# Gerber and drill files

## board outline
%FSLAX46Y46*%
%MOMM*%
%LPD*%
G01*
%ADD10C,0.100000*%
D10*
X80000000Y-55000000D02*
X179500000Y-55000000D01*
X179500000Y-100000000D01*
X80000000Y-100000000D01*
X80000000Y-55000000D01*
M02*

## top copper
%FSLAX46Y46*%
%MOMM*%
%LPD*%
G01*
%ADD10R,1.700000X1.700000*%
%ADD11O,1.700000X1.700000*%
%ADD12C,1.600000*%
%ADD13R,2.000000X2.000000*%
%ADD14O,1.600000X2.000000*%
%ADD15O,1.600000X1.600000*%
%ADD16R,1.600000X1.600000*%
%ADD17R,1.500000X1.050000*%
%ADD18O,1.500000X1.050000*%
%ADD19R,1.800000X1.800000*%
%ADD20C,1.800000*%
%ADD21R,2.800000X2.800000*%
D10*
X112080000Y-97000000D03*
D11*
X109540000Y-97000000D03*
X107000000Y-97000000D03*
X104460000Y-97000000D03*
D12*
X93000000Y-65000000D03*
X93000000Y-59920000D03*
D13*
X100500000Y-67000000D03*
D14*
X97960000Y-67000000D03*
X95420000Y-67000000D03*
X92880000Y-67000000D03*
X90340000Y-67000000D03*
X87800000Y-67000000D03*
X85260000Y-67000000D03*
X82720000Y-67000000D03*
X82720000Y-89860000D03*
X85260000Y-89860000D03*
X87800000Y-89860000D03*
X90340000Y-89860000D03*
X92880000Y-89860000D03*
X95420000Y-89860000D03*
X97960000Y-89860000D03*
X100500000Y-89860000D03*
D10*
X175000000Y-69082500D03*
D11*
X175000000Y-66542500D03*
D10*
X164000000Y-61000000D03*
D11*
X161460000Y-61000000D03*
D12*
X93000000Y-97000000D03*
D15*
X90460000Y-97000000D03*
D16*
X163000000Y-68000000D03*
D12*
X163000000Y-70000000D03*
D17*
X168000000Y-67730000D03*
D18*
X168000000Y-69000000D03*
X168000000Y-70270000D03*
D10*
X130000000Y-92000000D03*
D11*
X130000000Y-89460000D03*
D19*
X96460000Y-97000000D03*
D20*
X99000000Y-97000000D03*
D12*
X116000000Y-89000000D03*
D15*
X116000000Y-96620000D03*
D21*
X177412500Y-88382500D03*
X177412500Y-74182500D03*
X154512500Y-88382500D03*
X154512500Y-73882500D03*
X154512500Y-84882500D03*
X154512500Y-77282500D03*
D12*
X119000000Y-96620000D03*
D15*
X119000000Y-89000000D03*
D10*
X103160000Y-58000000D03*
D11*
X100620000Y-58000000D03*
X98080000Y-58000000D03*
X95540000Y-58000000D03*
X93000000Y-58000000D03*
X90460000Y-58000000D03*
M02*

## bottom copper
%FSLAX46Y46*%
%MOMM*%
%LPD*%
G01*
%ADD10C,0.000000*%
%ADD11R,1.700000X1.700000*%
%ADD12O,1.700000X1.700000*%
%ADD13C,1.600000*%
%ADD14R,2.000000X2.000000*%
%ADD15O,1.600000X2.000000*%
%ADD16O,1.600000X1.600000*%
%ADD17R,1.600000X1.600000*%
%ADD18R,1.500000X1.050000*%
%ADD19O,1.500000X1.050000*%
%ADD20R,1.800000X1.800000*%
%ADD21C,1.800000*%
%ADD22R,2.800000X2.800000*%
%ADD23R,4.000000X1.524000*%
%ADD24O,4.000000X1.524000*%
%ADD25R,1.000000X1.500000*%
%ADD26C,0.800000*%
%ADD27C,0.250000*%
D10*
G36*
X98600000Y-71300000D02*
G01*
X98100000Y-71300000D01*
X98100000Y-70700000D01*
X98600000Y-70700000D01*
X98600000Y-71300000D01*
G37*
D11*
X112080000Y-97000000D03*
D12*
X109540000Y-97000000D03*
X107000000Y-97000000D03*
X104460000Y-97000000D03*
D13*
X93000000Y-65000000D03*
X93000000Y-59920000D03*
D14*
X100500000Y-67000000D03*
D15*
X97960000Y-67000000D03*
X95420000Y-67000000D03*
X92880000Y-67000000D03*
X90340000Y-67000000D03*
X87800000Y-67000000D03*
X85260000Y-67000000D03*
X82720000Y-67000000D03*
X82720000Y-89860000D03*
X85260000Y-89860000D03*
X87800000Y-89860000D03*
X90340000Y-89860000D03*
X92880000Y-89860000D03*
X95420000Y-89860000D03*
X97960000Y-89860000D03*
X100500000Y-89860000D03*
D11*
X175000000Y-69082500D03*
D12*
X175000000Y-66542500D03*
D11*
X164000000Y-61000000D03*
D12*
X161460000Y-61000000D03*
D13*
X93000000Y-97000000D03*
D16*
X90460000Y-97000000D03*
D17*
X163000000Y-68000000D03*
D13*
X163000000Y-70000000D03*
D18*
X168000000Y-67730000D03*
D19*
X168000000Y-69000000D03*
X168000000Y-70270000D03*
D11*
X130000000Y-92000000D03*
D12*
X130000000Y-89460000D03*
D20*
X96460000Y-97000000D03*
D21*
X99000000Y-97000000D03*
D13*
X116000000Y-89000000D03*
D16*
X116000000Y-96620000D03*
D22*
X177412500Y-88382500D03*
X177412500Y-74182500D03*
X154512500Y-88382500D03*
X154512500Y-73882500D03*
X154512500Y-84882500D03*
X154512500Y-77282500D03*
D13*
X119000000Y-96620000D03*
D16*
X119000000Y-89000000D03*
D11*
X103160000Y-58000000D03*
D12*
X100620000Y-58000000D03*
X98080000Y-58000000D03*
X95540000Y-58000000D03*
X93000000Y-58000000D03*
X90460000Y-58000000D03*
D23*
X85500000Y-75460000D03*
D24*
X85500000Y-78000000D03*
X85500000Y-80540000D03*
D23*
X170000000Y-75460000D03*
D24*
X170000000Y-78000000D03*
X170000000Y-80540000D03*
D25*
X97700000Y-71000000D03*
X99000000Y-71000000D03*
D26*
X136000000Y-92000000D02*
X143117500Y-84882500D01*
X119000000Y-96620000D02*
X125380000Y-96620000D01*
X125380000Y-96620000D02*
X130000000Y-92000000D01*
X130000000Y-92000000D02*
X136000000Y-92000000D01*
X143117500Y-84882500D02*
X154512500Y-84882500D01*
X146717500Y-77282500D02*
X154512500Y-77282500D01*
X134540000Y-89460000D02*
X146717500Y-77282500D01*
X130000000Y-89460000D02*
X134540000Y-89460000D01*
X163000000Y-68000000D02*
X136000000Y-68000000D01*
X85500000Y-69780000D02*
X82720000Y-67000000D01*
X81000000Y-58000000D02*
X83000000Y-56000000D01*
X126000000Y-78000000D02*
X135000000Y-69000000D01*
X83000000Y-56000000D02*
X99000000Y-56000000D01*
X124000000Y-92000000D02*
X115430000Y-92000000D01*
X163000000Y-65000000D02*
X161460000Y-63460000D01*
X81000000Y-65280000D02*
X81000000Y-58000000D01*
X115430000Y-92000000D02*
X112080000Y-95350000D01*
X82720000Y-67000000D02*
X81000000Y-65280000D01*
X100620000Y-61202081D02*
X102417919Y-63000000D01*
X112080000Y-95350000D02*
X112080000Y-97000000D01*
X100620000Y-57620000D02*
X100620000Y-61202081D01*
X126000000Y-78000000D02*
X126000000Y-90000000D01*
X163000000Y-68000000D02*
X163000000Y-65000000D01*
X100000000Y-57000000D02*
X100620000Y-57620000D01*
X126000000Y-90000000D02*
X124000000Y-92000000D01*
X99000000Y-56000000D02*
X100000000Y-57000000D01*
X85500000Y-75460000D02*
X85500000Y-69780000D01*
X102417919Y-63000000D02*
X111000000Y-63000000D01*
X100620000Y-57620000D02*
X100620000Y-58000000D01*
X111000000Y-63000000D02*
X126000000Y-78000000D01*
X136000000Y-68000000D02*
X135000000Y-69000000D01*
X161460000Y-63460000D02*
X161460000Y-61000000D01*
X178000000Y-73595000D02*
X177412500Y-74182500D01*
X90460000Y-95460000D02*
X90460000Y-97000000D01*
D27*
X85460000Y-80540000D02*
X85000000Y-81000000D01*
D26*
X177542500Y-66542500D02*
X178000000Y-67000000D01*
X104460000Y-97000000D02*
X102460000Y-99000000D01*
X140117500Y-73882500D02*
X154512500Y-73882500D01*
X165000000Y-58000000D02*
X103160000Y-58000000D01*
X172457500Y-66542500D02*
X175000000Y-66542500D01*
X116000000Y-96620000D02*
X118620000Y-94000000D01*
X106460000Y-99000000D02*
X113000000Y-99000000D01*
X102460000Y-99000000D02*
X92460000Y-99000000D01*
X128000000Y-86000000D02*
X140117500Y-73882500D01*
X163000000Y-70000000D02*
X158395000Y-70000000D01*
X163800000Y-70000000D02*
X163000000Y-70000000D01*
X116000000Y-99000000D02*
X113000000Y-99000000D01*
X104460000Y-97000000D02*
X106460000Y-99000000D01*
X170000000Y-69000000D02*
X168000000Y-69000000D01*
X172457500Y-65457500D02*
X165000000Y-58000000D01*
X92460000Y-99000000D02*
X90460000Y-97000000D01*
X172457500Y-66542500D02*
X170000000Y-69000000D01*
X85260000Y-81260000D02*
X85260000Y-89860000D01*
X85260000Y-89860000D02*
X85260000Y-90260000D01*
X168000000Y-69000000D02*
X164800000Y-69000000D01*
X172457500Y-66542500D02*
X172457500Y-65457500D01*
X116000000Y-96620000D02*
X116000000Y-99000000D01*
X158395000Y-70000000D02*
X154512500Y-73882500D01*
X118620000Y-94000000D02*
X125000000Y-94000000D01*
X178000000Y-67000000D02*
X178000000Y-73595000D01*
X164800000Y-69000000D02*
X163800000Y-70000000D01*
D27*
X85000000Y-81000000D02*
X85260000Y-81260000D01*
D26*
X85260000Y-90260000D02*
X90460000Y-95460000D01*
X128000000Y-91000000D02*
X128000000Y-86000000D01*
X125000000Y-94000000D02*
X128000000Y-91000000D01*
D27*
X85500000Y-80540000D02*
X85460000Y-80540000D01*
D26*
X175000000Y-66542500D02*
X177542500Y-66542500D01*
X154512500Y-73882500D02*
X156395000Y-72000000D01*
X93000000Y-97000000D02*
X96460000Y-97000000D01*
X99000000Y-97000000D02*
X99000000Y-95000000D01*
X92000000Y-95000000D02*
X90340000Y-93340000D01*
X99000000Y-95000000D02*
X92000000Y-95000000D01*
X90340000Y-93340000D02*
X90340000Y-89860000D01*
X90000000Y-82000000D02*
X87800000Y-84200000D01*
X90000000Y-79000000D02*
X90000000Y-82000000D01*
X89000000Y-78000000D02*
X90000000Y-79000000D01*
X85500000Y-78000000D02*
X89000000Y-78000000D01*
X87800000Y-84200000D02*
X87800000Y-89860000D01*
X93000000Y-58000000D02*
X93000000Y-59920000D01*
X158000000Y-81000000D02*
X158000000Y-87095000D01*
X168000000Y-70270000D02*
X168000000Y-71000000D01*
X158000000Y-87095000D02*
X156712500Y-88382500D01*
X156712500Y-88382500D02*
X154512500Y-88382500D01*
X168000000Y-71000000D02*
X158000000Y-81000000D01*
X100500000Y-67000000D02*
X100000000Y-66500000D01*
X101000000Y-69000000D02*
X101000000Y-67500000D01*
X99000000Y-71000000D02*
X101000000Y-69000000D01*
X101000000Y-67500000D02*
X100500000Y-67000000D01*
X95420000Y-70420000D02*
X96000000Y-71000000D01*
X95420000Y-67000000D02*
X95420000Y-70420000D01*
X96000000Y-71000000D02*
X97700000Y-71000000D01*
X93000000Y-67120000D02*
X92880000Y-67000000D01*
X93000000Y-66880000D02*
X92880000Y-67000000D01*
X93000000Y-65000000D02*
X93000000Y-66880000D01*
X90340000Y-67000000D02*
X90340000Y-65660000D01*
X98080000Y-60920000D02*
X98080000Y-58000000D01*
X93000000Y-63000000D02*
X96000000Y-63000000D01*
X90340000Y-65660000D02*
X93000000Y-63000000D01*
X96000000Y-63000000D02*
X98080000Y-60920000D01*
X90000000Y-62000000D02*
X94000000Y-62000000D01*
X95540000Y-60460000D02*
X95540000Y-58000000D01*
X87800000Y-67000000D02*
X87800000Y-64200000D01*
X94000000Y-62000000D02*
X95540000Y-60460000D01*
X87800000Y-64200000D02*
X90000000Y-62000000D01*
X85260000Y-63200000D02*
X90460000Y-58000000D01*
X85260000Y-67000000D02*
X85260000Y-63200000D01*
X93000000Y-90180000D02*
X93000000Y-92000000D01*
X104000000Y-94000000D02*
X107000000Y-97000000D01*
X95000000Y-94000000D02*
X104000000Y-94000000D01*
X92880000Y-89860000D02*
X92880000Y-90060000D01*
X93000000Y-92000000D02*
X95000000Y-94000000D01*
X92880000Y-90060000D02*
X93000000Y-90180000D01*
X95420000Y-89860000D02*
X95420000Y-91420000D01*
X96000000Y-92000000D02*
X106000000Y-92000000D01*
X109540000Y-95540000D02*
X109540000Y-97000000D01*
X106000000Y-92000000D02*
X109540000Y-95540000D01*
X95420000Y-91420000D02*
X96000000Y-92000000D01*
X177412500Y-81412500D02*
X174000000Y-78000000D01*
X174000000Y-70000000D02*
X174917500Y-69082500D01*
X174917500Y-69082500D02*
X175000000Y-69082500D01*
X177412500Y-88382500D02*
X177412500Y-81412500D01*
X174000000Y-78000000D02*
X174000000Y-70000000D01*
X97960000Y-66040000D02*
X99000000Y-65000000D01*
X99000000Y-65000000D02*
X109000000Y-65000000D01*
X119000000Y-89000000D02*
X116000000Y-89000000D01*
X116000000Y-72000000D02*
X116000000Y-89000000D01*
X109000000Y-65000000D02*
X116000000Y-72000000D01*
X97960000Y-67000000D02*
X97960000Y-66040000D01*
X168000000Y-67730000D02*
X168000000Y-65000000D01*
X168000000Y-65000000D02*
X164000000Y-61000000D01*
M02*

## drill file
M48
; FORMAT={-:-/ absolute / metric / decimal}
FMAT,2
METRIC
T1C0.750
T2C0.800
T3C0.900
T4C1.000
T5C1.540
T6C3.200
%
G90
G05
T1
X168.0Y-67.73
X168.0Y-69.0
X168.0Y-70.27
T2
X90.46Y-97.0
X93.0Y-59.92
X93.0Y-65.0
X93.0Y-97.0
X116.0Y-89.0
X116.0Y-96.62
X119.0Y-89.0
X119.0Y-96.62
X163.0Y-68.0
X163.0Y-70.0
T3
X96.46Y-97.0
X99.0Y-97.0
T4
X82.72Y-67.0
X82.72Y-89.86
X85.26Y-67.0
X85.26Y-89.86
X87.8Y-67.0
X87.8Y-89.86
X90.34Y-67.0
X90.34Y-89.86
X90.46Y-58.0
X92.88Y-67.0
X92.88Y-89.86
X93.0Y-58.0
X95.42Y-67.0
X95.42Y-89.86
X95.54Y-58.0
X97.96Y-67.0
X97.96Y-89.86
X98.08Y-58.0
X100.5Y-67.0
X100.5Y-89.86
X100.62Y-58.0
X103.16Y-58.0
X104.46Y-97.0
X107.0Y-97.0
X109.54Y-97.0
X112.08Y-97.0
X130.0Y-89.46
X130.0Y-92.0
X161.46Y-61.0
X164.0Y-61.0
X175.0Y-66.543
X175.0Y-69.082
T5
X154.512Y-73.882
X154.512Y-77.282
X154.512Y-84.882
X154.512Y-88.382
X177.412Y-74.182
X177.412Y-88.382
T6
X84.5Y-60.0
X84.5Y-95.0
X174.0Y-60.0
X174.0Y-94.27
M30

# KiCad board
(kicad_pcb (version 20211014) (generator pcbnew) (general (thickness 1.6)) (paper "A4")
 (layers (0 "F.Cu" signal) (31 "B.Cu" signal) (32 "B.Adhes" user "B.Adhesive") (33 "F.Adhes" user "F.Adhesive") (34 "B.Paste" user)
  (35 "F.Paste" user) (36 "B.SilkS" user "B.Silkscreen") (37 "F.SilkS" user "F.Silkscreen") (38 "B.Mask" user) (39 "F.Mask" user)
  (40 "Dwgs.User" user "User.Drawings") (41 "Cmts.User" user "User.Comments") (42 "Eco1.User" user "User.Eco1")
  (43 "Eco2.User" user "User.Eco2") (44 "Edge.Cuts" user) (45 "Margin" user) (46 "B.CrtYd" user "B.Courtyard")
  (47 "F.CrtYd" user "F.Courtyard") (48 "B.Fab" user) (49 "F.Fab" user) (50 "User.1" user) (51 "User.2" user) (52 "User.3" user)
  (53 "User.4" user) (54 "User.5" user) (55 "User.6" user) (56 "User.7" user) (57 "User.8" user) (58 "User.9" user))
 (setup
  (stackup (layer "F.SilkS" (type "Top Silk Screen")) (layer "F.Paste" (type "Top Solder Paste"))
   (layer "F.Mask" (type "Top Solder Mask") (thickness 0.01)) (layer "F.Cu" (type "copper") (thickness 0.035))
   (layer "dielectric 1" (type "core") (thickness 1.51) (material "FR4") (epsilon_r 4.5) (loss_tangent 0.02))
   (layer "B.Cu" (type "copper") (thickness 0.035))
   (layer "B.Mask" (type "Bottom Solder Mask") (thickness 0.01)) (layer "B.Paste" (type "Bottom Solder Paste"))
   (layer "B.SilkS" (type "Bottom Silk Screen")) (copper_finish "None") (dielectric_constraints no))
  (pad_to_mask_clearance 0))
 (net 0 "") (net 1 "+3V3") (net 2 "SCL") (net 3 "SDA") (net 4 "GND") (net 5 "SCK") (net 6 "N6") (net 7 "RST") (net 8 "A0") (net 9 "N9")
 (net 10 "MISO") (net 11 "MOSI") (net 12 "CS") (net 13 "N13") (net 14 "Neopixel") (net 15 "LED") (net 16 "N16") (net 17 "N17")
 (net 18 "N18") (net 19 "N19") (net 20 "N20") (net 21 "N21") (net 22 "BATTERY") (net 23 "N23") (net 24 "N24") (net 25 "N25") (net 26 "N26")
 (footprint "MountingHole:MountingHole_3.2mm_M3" (layer "F.Cu") (at 174 60)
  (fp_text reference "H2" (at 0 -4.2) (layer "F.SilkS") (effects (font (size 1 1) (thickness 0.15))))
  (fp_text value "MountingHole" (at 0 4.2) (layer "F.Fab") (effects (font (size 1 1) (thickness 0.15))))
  (pad "" np_thru_hole circle (at 0 0) (size 3.2 3.2) (drill 3.2) (layers *.Cu *.Mask)))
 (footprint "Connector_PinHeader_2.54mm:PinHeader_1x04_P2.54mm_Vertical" (layer "F.Cu") (at 112.08 97 -90)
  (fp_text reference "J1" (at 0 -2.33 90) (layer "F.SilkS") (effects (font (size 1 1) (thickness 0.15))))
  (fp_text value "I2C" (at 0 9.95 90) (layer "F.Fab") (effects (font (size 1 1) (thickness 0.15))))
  (pad "1" thru_hole rect (at 0 0 270) (size 1.7 1.7) (drill 1) (layers *.Cu *.Mask) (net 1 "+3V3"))
  (pad "2" thru_hole oval (at 0 2.54 270) (size 1.7 1.7) (drill 1) (layers *.Cu *.Mask) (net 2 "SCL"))
  (pad "3" thru_hole oval (at 0 5.08 270) (size 1.7 1.7) (drill 1) (layers *.Cu *.Mask) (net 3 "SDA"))
  (pad "4" thru_hole oval (at 0 7.62 270) (size 1.7 1.7) (drill 1) (layers *.Cu *.Mask) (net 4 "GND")))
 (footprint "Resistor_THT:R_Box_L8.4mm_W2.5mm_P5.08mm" (layer "F.Cu") (at 93 65 90)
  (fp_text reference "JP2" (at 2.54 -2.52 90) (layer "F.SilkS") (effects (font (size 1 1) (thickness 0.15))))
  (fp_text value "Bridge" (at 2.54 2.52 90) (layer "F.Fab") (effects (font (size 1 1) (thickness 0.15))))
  (pad "1" thru_hole circle (at 0 0 90) (size 1.6 1.6) (drill 0.8) (layers *.Cu *.Mask) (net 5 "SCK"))
  (pad "2" thru_hole circle (at 5.08 0 90) (size 1.6 1.6) (drill 0.8) (layers *.Cu *.Mask) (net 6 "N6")))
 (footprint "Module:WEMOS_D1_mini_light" (layer "F.Cu") (at 100.5 67 -90)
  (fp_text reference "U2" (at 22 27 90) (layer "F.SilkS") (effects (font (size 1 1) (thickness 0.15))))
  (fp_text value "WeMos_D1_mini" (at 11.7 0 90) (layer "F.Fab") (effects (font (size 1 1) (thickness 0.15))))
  (pad "1" thru_hole rect (at 0 0 270) (size 2 2) (drill 1) (layers *.Cu *.Mask) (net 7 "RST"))
  (pad "2" thru_hole oval (at 0 2.54 270) (size 2 1.6) (drill 1) (layers *.Cu *.Mask) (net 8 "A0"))
  (pad "3" thru_hole oval (at 0 5.08 270) (size 2 1.6) (drill 1) (layers *.Cu *.Mask) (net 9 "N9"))
  (pad "4" thru_hole oval (at 0 7.62 270) (size 2 1.6) (drill 1) (layers *.Cu *.Mask) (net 5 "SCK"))
  (pad "5" thru_hole oval (at 0 10.16 270) (size 2 1.6) (drill 1) (layers *.Cu *.Mask) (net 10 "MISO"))
  (pad "6" thru_hole oval (at 0 12.7 270) (size 2 1.6) (drill 1) (layers *.Cu *.Mask) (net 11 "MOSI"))
  (pad "7" thru_hole oval (at 0 15.24 270) (size 2 1.6) (drill 1) (layers *.Cu *.Mask) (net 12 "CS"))
  (pad "8" thru_hole oval (at 0 17.78 270) (size 2 1.6) (drill 1) (layers *.Cu *.Mask) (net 1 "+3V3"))
  (pad "9" thru_hole oval (at 22.86 17.78 270) (size 2 1.6) (drill 1) (layers *.Cu *.Mask) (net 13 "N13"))
  (pad "10" thru_hole oval (at 22.86 15.24 270) (size 2 1.6) (drill 1) (layers *.Cu *.Mask) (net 4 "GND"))
  (pad "11" thru_hole oval (at 22.86 12.7 270) (size 2 1.6) (drill 1) (layers *.Cu *.Mask) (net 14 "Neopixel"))
  (pad "12" thru_hole oval (at 22.86 10.16 270) (size 2 1.6) (drill 1) (layers *.Cu *.Mask) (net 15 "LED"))
  (pad "13" thru_hole oval (at 22.86 7.62 270) (size 2 1.6) (drill 1) (layers *.Cu *.Mask) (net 3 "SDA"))
  (pad "14" thru_hole oval (at 22.86 5.08 270) (size 2 1.6) (drill 1) (layers *.Cu *.Mask) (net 2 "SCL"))
  (pad "15" thru_hole oval (at 22.86 2.54 270) (size 2 1.6) (drill 1) (layers *.Cu *.Mask) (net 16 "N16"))
  (pad "16" thru_hole oval (at 22.86 0 270) (size 2 1.6) (drill 1) (layers *.Cu *.Mask) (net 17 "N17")))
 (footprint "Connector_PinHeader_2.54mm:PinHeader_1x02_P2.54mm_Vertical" (layer "F.Cu") (at 175 69.0825 180)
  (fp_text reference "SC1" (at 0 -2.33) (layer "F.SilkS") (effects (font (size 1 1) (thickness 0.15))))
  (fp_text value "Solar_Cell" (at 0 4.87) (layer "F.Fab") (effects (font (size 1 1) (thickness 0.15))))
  (pad "1" thru_hole rect (at 0 0 180) (size 1.7 1.7) (drill 1) (layers *.Cu *.Mask) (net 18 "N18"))
  (pad "2" thru_hole oval (at 0 2.54 180) (size 1.7 1.7) (drill 1) (layers *.Cu *.Mask) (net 4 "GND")))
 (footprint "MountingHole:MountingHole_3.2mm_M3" (layer "F.Cu") (at 84.5 95)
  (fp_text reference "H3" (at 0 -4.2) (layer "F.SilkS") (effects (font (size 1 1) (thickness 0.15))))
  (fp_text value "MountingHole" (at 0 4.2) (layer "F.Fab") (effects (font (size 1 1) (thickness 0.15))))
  (pad "" np_thru_hole circle (at 0 0) (size 3.2 3.2) (drill 3.2) (layers *.Cu *.Mask)))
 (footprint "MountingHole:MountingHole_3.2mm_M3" (layer "F.Cu") (at 174 94.27)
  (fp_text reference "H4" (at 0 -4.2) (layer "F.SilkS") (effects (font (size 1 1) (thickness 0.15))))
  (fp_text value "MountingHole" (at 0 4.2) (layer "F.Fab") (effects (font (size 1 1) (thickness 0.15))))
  (pad "" np_thru_hole circle (at 0 0) (size 3.2 3.2) (drill 3.2) (layers *.Cu *.Mask)))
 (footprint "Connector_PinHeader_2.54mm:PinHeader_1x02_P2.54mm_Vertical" (layer "F.Cu") (at 164 61 -90)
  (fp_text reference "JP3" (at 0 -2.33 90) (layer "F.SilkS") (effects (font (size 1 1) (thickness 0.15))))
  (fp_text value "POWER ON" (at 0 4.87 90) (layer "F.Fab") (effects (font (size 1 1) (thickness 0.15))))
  (pad "1" thru_hole rect (at 0 0 270) (size 1.7 1.7) (drill 1) (layers *.Cu *.Mask) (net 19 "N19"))
  (pad "2" thru_hole oval (at 0 2.54 270) (size 1.7 1.7) (drill 1) (layers *.Cu *.Mask) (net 1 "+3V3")))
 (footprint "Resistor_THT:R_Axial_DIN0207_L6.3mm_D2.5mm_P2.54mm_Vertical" (layer "F.Cu") (at 93 97 180)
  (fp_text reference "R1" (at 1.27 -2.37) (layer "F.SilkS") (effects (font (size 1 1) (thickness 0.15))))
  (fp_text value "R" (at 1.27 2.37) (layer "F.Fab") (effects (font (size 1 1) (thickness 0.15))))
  (pad "1" thru_hole circle (at 0 0 180) (size 1.6 1.6) (drill 0.8) (layers *.Cu *.Mask) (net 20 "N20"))
  (pad "2" thru_hole oval (at 2.54 0 180) (size 1.6 1.6) (drill 0.8) (layers *.Cu *.Mask) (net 4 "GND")))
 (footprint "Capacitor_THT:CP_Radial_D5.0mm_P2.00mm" (layer "F.Cu") (at 163 68 -90)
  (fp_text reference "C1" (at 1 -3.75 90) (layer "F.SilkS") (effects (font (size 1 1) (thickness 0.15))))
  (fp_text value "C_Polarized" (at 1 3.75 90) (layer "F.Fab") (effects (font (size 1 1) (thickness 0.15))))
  (pad "1" thru_hole rect (at 0 0 270) (size 1.6 1.6) (drill 0.8) (layers *.Cu *.Mask) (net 1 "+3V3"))
  (pad "2" thru_hole circle (at 2 0 270) (size 1.6 1.6) (drill 0.8) (layers *.Cu *.Mask) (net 4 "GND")))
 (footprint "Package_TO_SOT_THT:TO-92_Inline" (layer "F.Cu") (at 168 67.73 -90)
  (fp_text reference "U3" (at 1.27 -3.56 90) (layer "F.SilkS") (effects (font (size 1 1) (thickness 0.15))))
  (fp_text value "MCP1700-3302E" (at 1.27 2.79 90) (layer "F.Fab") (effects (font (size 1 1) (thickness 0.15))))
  (pad "1" thru_hole rect (at 0 0 270) (size 1.05 1.5) (drill 0.75) (layers *.Cu *.Mask) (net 19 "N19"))
  (pad "2" thru_hole oval (at 1.27 0 270) (size 1.05 1.5) (drill 0.75) (layers *.Cu *.Mask) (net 4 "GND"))
  (pad "3" thru_hole oval (at 2.54 0 270) (size 1.05 1.5) (drill 0.75) (layers *.Cu *.Mask) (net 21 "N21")))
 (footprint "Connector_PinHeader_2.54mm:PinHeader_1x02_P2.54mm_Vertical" (layer "F.Cu") (at 130 92 180)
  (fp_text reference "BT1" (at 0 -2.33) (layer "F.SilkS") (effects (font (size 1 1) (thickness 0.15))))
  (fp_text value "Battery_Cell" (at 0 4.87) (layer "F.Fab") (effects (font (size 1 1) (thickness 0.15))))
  (pad "1" thru_hole rect (at 0 0 180) (size 1.7 1.7) (drill 1) (layers *.Cu *.Mask) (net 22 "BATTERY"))
  (pad "2" thru_hole oval (at 0 2.54 180) (size 1.7 1.7) (drill 1) (layers *.Cu *.Mask) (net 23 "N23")))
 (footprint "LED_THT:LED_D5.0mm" (layer "F.Cu") (at 96.46 97)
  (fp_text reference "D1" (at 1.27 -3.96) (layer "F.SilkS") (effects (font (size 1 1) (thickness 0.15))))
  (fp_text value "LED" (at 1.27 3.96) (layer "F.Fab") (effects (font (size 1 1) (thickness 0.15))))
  (pad "1" thru_hole rect (at 0 0) (size 1.8 1.8) (drill 0.9) (layers *.Cu *.Mask) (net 20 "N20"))
  (pad "2" thru_hole circle (at 2.54 0) (size 1.8 1.8) (drill 0.9) (layers *.Cu *.Mask) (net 15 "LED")))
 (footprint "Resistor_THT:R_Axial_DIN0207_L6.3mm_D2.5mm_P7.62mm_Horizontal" (layer "F.Cu") (at 116 89 -90)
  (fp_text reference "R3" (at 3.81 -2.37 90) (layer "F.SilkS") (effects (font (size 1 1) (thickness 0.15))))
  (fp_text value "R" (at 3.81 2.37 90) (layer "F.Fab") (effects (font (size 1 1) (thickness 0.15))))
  (pad "1" thru_hole circle (at 0 0 270) (size 1.6 1.6) (drill 0.8) (layers *.Cu *.Mask) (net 8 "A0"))
  (pad "2" thru_hole oval (at 7.62 0 270) (size 1.6 1.6) (drill 0.8) (layers *.Cu *.Mask) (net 4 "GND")))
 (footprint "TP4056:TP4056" (layer "F.Cu") (at 179.1125 90.0825 180)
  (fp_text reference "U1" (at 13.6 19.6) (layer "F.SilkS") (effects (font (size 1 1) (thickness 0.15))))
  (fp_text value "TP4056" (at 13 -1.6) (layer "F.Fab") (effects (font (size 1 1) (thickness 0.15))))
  (pad "1" thru_hole rect locked (at 1.7 1.7 180) (size 2.8 2.8) (drill 1.54) (layers *.Cu *.Mask) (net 18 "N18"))
  (pad "2" thru_hole rect locked (at 1.7 15.9 180) (size 2.8 2.8) (drill 1.54) (layers *.Cu *.Mask) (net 4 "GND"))
  (pad "3" thru_hole rect locked (at 24.6 1.7 180) (size 2.8 2.8) (drill 1.54) (layers *.Cu *.Mask) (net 21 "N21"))
  (pad "4" thru_hole rect locked (at 24.6 16.2 180) (size 2.8 2.8) (drill 1.54) (layers *.Cu *.Mask) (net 4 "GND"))
  (pad "5" thru_hole rect locked (at 24.6 5.2 180) (size 2.8 2.8) (drill 1.54) (layers *.Cu *.Mask) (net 22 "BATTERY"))
  (pad "6" thru_hole rect locked (at 24.6 12.8 180) (size 2.8 2.8) (drill 1.54) (layers *.Cu *.Mask) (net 23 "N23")))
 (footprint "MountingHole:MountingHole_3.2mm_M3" (layer "F.Cu") (at 84.5 60)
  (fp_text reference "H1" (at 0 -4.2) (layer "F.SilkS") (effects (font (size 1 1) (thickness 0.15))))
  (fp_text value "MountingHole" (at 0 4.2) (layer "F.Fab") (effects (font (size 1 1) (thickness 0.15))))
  (pad "" np_thru_hole circle (at 0 0) (size 3.2 3.2) (drill 3.2) (layers *.Cu *.Mask)))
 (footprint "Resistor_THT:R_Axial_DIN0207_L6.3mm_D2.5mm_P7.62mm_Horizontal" (layer "F.Cu") (at 119 96.62 90)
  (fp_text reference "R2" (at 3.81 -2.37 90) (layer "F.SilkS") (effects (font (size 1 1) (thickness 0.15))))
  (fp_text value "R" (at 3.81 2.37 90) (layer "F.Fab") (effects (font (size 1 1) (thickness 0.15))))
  (pad "1" thru_hole circle (at 0 0 90) (size 1.6 1.6) (drill 0.8) (layers *.Cu *.Mask) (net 22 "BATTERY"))
  (pad "2" thru_hole oval (at 7.62 0 90) (size 1.6 1.6) (drill 0.8) (layers *.Cu *.Mask) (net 8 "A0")))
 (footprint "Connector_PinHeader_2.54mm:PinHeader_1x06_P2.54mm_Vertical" (layer "F.Cu") (at 103.16 58 -90)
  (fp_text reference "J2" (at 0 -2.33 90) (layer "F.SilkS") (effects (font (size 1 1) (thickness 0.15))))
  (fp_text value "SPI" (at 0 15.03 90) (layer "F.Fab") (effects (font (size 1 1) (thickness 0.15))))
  (pad "1" thru_hole rect (at 0 0 270) (size 1.7 1.7) (drill 1) (layers *.Cu *.Mask) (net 4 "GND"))
  (pad "2" thru_hole oval (at 0 2.54 270) (size 1.7 1.7) (drill 1) (layers *.Cu *.Mask) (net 1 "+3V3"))
  (pad "3" thru_hole oval (at 0 5.08 270) (size 1.7 1.7) (drill 1) (layers *.Cu *.Mask) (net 10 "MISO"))
  (pad "4" thru_hole oval (at 0 7.62 270) (size 1.7 1.7) (drill 1) (layers *.Cu *.Mask) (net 11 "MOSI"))
  (pad "5" thru_hole oval (at 0 10.16 270) (size 1.7 1.7) (drill 1) (layers *.Cu *.Mask) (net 6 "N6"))
  (pad "6" thru_hole oval (at 0 12.7 270) (size 1.7 1.7) (drill 1) (layers *.Cu *.Mask) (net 12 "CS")))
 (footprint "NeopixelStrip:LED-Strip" (layer "B.Cu") (at 85.5 78 -90)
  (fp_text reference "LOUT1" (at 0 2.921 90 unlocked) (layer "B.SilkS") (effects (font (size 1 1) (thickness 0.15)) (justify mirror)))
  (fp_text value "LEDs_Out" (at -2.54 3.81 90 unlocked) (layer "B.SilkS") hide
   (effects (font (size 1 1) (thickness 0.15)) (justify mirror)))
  (pad "1" connect rect locked (at -2.54 0 270) (size 1.524 4) (layers "B.Cu" "B.Mask") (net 1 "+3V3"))
  (pad "2" connect oval locked (at 0 0 270) (size 1.524 4) (layers "B.Cu" "B.Mask") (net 14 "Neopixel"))
  (pad "3" connect oval locked (at 2.54 0 270) (size 1.524 4) (layers "B.Cu" "B.Mask") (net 4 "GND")))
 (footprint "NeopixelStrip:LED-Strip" (layer "B.Cu") (at 170 78 -90)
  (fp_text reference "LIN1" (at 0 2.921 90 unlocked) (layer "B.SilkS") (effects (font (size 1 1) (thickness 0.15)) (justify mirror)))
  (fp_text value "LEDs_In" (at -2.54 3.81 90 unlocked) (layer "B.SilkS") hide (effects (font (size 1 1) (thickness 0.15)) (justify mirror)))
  (pad "1" connect rect locked (at -2.54 0 270) (size 1.524 4) (layers "B.Cu" "B.Mask") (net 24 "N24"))
  (pad "2" connect oval locked (at 0 0 270) (size 1.524 4) (layers "B.Cu" "B.Mask") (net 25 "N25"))
  (pad "3" connect oval locked (at 2.54 0 270) (size 1.524 4) (layers "B.Cu" "B.Mask") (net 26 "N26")))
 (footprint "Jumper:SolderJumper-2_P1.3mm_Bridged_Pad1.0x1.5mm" (layer "B.Cu") (at 98.35 71)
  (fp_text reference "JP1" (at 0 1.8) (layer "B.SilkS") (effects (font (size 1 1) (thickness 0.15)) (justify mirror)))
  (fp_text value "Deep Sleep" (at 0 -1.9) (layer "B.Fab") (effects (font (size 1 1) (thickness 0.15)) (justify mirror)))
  (fp_poly (pts (xy -0.25 0.3) (xy 0.25 0.3) (xy 0.25 -0.3) (xy -0.25 -0.3)) (layer "B.Cu") (width 0) (fill solid))
  (pad "1" smd rect (at -0.65 0) (size 1 1.5) (layers "B.Cu" "B.Mask") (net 9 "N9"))
  (pad "2" smd rect (at 0.65 0) (size 1 1.5) (layers "B.Cu" "B.Mask") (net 7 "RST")))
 (gr_rect (start 80 55) (end 179.5 100) (layer "Edge.Cuts") (width 0.1) (fill none))
 (segment (start 136 92) (end 143.1175 84.8825) (width 0.8) (layer "B.Cu") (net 22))
 (segment (start 119 96.62) (end 125.38 96.62) (width 0.8) (layer "B.Cu") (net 22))
 (segment (start 125.38 96.62) (end 130 92) (width 0.8) (layer "B.Cu") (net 22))
 (segment (start 130 92) (end 136 92) (width 0.8) (layer "B.Cu") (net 22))
 (segment (start 143.1175 84.8825) (end 154.5125 84.8825) (width 0.8) (layer "B.Cu") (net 22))
 (segment (start 146.7175 77.2825) (end 154.5125 77.2825) (width 0.8) (layer "B.Cu") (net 23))
 (segment (start 134.54 89.46) (end 146.7175 77.2825) (width 0.8) (layer "B.Cu") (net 23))
 (segment (start 130 89.46) (end 134.54 89.46) (width 0.8) (layer "B.Cu") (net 23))
 (segment (start 163 68) (end 136 68) (width 0.8) (layer "B.Cu") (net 1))
 (segment (start 85.5 69.78) (end 82.72 67) (width 0.8) (layer "B.Cu") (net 1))
 (segment (start 81 58) (end 83 56) (width 0.8) (layer "B.Cu") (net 1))
 (segment (start 126 78) (end 135 69) (width 0.8) (layer "B.Cu") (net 1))
 (segment (start 83 56) (end 99 56) (width 0.8) (layer "B.Cu") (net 1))
 (segment (start 124 92) (end 115.43 92) (width 0.8) (layer "B.Cu") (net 1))
 (segment (start 163 65) (end 161.46 63.46) (width 0.8) (layer "B.Cu") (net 1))
 (segment (start 81 65.28) (end 81 58) (width 0.8) (layer "B.Cu") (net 1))
 (segment (start 115.43 92) (end 112.08 95.35) (width 0.8) (layer "B.Cu") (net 1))
 (segment (start 82.72 67) (end 81 65.28) (width 0.8) (layer "B.Cu") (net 1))
 (segment (start 100.62 61.202081) (end 102.417919 63) (width 0.8) (layer "B.Cu") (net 1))
 (segment (start 112.08 95.35) (end 112.08 97) (width 0.8) (layer "B.Cu") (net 1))
 (segment (start 100.62 57.62) (end 100.62 61.202081) (width 0.8) (layer "B.Cu") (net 1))
 (segment (start 126 78) (end 126 90) (width 0.8) (layer "B.Cu") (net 1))
 (segment (start 163 68) (end 163 65) (width 0.8) (layer "B.Cu") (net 1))
 (segment (start 100 57) (end 100.62 57.62) (width 0.8) (layer "B.Cu") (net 1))
 (segment (start 126 90) (end 124 92) (width 0.8) (layer "B.Cu") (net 1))
 (segment (start 99 56) (end 100 57) (width 0.8) (layer "B.Cu") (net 1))
 (segment (start 85.5 75.46) (end 85.5 69.78) (width 0.8) (layer "B.Cu") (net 1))
 (segment (start 102.417919 63) (end 111 63) (width 0.8) (layer "B.Cu") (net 1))
 (segment (start 100.62 57.62) (end 100.62 58) (width 0.8) (layer "B.Cu") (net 1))
 (segment (start 111 63) (end 126 78) (width 0.8) (layer "B.Cu") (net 1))
 (segment (start 136 68) (end 135 69) (width 0.8) (layer "B.Cu") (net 1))
 (segment (start 161.46 63.46) (end 161.46 61) (width 0.8) (layer "B.Cu") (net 1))
 (segment (start 178 73.595) (end 177.4125 74.1825) (width 0.8) (layer "B.Cu") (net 4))
 (segment (start 90.46 95.46) (end 90.46 97) (width 0.8) (layer "B.Cu") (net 4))
 (segment (start 85.46 80.54) (end 85 81) (width 0.25) (layer "B.Cu") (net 4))
 (segment (start 177.5425 66.5425) (end 178 67) (width 0.8) (layer "B.Cu") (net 4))
 (segment (start 104.46 97) (end 102.46 99) (width 0.8) (layer "B.Cu") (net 4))
 (segment (start 140.1175 73.8825) (end 154.5125 73.8825) (width 0.8) (layer "B.Cu") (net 4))
 (segment (start 165 58) (end 103.16 58) (width 0.8) (layer "B.Cu") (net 4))
 (segment (start 172.4575 66.5425) (end 175 66.5425) (width 0.8) (layer "B.Cu") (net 4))
 (segment (start 116 96.62) (end 118.62 94) (width 0.8) (layer "B.Cu") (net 4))
 (segment (start 106.46 99) (end 113 99) (width 0.8) (layer "B.Cu") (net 4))
 (segment (start 102.46 99) (end 92.46 99) (width 0.8) (layer "B.Cu") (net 4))
 (segment (start 128 86) (end 140.1175 73.8825) (width 0.8) (layer "B.Cu") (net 4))
 (segment (start 163 70) (end 158.395 70) (width 0.8) (layer "B.Cu") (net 4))
 (segment (start 163.8 70) (end 163 70) (width 0.8) (layer "B.Cu") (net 4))
 (segment (start 116 99) (end 113 99) (width 0.8) (layer "B.Cu") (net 4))
 (segment (start 104.46 97) (end 106.46 99) (width 0.8) (layer "B.Cu") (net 4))
 (segment (start 170 69) (end 168 69) (width 0.8) (layer "B.Cu") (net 4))
 (segment (start 172.4575 65.4575) (end 165 58) (width 0.8) (layer "B.Cu") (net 4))
 (segment (start 92.46 99) (end 90.46 97) (width 0.8) (layer "B.Cu") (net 4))
 (segment (start 172.4575 66.5425) (end 170 69) (width 0.8) (layer "B.Cu") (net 4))
 (segment (start 85.26 81.26) (end 85.26 89.86) (width 0.8) (layer "B.Cu") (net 4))
 (segment (start 85.26 89.86) (end 85.26 90.26) (width 0.8) (layer "B.Cu") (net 4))
 (segment (start 168 69) (end 164.8 69) (width 0.8) (layer "B.Cu") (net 4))
 (segment (start 172.4575 66.5425) (end 172.4575 65.4575) (width 0.8) (layer "B.Cu") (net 4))
 (segment (start 116 96.62) (end 116 99) (width 0.8) (layer "B.Cu") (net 4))
 (segment (start 158.395 70) (end 154.5125 73.8825) (width 0.8) (layer "B.Cu") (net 4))
 (segment (start 118.62 94) (end 125 94) (width 0.8) (layer "B.Cu") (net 4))
 (segment (start 178 67) (end 178 73.595) (width 0.8) (layer "B.Cu") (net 4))
 (segment (start 164.8 69) (end 163.8 70) (width 0.8) (layer "B.Cu") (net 4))
 (segment (start 85 81) (end 85.26 81.26) (width 0.25) (layer "B.Cu") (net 4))
 (segment (start 85.26 90.26) (end 90.46 95.46) (width 0.8) (layer "B.Cu") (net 4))
 (segment (start 128 91) (end 128 86) (width 0.8) (layer "B.Cu") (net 4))
 (segment (start 125 94) (end 128 91) (width 0.8) (layer "B.Cu") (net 4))
 (segment (start 85.5 80.54) (end 85.46 80.54) (width 0.25) (layer "B.Cu") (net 4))
 (segment (start 175 66.5425) (end 177.5425 66.5425) (width 0.8) (layer "B.Cu") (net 4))
 (segment (start 154.5125 73.8825) (end 156.395 72) (width 0.8) (layer "B.Cu") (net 4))
 (segment (start 93 97) (end 96.46 97) (width 0.8) (layer "B.Cu") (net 20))
 (segment (start 99 97) (end 99 95) (width 0.8) (layer "B.Cu") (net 15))
 (segment (start 92 95) (end 90.34 93.34) (width 0.8) (layer "B.Cu") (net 15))
 (segment (start 99 95) (end 92 95) (width 0.8) (layer "B.Cu") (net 15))
 (segment (start 90.34 93.34) (end 90.34 89.86) (width 0.8) (layer "B.Cu") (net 15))
 (segment (start 90 82) (end 87.8 84.2) (width 0.8) (layer "B.Cu") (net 14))
 (segment (start 90 79) (end 90 82) (width 0.8) (layer "B.Cu") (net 14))
 (segment (start 89 78) (end 90 79) (width 0.8) (layer "B.Cu") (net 14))
 (segment (start 85.5 78) (end 89 78) (width 0.8) (layer "B.Cu") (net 14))
 (segment (start 87.8 84.2) (end 87.8 89.86) (width 0.8) (layer "B.Cu") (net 14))
 (segment (start 93 58) (end 93 59.92) (width 0.8) (layer "B.Cu") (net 6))
 (segment (start 158 81) (end 158 87.095) (width 0.8) (layer "B.Cu") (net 21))
 (segment (start 168 70.27) (end 168 71) (width 0.8) (layer "B.Cu") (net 21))
 (segment (start 158 87.095) (end 156.7125 88.3825) (width 0.8) (layer "B.Cu") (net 21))
 (segment (start 156.7125 88.3825) (end 154.5125 88.3825) (width 0.8) (layer "B.Cu") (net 21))
 (segment (start 168 71) (end 158 81) (width 0.8) (layer "B.Cu") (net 21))
 (segment (start 100.5 67) (end 100 66.5) (width 0.8) (layer "B.Cu") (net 7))
 (segment (start 101 69) (end 101 67.5) (width 0.8) (layer "B.Cu") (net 7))
 (segment (start 99 71) (end 101 69) (width 0.8) (layer "B.Cu") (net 7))
 (segment (start 101 67.5) (end 100.5 67) (width 0.8) (layer "B.Cu") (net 7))
 (segment (start 95.42 70.42) (end 96 71) (width 0.8) (layer "B.Cu") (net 9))
 (segment (start 95.42 67) (end 95.42 70.42) (width 0.8) (layer "B.Cu") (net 9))
 (segment (start 96 71) (end 97.7 71) (width 0.8) (layer "B.Cu") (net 9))
 (segment (start 93 67.12) (end 92.88 67) (width 0.8) (layer "B.Cu") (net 5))
 (segment (start 93 66.88) (end 92.88 67) (width 0.8) (layer "B.Cu") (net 5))
 (segment (start 93 65) (end 93 66.88) (width 0.8) (layer "B.Cu") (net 5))
 (segment (start 90.34 67) (end 90.34 65.66) (width 0.8) (layer "B.Cu") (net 10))
 (segment (start 98.08 60.92) (end 98.08 58) (width 0.8) (layer "B.Cu") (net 10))
 (segment (start 93 63) (end 96 63) (width 0.8) (layer "B.Cu") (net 10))
 (segment (start 90.34 65.66) (end 93 63) (width 0.8) (layer "B.Cu") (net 10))
 (segment (start 96 63) (end 98.08 60.92) (width 0.8) (layer "B.Cu") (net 10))
 (segment (start 90 62) (end 94 62) (width 0.8) (layer "B.Cu") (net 11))
 (segment (start 95.54 60.46) (end 95.54 58) (width 0.8) (layer "B.Cu") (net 11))
 (segment (start 87.8 67) (end 87.8 64.2) (width 0.8) (layer "B.Cu") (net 11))
 (segment (start 94 62) (end 95.54 60.46) (width 0.8) (layer "B.Cu") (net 11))
 (segment (start 87.8 64.2) (end 90 62) (width 0.8) (layer "B.Cu") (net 11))
 (segment (start 85.26 63.2) (end 90.46 58) (width 0.8) (layer "B.Cu") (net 12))
 (segment (start 85.26 67) (end 85.26 63.2) (width 0.8) (layer "B.Cu") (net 12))
 (segment (start 93 90.18) (end 93 92) (width 0.8) (layer "B.Cu") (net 3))
 (segment (start 104 94) (end 107 97) (width 0.8) (layer "B.Cu") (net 3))
 (segment (start 95 94) (end 104 94) (width 0.8) (layer "B.Cu") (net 3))
 (segment (start 92.88 89.86) (end 92.88 90.06) (width 0.8) (layer "B.Cu") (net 3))
 (segment (start 93 92) (end 95 94) (width 0.8) (layer "B.Cu") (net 3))
 (segment (start 92.88 90.06) (end 93 90.18) (width 0.8) (layer "B.Cu") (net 3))
 (segment (start 95.42 89.86) (end 95.42 91.42) (width 0.8) (layer "B.Cu") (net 2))
 (segment (start 96 92) (end 106 92) (width 0.8) (layer "B.Cu") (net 2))
 (segment (start 109.54 95.54) (end 109.54 97) (width 0.8) (layer "B.Cu") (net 2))
 (segment (start 106 92) (end 109.54 95.54) (width 0.8) (layer "B.Cu") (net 2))
 (segment (start 95.42 91.42) (end 96 92) (width 0.8) (layer "B.Cu") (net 2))
 (segment (start 177.4125 81.4125) (end 174 78) (width 0.8) (layer "B.Cu") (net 18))
 (segment (start 174 70) (end 174.9175 69.0825) (width 0.8) (layer "B.Cu") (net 18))
 (segment (start 174.9175 69.0825) (end 175 69.0825) (width 0.8) (layer "B.Cu") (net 18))
 (segment (start 177.4125 88.3825) (end 177.4125 81.4125) (width 0.8) (layer "B.Cu") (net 18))
 (segment (start 174 78) (end 174 70) (width 0.8) (layer "B.Cu") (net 18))
 (segment (start 97.96 66.04) (end 99 65) (width 0.8) (layer "B.Cu") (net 8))
 (segment (start 99 65) (end 109 65) (width 0.8) (layer "B.Cu") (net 8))
 (segment (start 119 89) (end 116 89) (width 0.8) (layer "B.Cu") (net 8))
 (segment (start 116 72) (end 116 89) (width 0.8) (layer "B.Cu") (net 8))
 (segment (start 109 65) (end 116 72) (width 0.8) (layer "B.Cu") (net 8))
 (segment (start 97.96 67) (end 97.96 66.04) (width 0.8) (layer "B.Cu") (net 8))
 (segment (start 168 67.73) (end 168 65) (width 0.8) (layer "B.Cu") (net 19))
 (segment (start 168 65) (end 164 61) (width 0.8) (layer "B.Cu") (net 19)))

